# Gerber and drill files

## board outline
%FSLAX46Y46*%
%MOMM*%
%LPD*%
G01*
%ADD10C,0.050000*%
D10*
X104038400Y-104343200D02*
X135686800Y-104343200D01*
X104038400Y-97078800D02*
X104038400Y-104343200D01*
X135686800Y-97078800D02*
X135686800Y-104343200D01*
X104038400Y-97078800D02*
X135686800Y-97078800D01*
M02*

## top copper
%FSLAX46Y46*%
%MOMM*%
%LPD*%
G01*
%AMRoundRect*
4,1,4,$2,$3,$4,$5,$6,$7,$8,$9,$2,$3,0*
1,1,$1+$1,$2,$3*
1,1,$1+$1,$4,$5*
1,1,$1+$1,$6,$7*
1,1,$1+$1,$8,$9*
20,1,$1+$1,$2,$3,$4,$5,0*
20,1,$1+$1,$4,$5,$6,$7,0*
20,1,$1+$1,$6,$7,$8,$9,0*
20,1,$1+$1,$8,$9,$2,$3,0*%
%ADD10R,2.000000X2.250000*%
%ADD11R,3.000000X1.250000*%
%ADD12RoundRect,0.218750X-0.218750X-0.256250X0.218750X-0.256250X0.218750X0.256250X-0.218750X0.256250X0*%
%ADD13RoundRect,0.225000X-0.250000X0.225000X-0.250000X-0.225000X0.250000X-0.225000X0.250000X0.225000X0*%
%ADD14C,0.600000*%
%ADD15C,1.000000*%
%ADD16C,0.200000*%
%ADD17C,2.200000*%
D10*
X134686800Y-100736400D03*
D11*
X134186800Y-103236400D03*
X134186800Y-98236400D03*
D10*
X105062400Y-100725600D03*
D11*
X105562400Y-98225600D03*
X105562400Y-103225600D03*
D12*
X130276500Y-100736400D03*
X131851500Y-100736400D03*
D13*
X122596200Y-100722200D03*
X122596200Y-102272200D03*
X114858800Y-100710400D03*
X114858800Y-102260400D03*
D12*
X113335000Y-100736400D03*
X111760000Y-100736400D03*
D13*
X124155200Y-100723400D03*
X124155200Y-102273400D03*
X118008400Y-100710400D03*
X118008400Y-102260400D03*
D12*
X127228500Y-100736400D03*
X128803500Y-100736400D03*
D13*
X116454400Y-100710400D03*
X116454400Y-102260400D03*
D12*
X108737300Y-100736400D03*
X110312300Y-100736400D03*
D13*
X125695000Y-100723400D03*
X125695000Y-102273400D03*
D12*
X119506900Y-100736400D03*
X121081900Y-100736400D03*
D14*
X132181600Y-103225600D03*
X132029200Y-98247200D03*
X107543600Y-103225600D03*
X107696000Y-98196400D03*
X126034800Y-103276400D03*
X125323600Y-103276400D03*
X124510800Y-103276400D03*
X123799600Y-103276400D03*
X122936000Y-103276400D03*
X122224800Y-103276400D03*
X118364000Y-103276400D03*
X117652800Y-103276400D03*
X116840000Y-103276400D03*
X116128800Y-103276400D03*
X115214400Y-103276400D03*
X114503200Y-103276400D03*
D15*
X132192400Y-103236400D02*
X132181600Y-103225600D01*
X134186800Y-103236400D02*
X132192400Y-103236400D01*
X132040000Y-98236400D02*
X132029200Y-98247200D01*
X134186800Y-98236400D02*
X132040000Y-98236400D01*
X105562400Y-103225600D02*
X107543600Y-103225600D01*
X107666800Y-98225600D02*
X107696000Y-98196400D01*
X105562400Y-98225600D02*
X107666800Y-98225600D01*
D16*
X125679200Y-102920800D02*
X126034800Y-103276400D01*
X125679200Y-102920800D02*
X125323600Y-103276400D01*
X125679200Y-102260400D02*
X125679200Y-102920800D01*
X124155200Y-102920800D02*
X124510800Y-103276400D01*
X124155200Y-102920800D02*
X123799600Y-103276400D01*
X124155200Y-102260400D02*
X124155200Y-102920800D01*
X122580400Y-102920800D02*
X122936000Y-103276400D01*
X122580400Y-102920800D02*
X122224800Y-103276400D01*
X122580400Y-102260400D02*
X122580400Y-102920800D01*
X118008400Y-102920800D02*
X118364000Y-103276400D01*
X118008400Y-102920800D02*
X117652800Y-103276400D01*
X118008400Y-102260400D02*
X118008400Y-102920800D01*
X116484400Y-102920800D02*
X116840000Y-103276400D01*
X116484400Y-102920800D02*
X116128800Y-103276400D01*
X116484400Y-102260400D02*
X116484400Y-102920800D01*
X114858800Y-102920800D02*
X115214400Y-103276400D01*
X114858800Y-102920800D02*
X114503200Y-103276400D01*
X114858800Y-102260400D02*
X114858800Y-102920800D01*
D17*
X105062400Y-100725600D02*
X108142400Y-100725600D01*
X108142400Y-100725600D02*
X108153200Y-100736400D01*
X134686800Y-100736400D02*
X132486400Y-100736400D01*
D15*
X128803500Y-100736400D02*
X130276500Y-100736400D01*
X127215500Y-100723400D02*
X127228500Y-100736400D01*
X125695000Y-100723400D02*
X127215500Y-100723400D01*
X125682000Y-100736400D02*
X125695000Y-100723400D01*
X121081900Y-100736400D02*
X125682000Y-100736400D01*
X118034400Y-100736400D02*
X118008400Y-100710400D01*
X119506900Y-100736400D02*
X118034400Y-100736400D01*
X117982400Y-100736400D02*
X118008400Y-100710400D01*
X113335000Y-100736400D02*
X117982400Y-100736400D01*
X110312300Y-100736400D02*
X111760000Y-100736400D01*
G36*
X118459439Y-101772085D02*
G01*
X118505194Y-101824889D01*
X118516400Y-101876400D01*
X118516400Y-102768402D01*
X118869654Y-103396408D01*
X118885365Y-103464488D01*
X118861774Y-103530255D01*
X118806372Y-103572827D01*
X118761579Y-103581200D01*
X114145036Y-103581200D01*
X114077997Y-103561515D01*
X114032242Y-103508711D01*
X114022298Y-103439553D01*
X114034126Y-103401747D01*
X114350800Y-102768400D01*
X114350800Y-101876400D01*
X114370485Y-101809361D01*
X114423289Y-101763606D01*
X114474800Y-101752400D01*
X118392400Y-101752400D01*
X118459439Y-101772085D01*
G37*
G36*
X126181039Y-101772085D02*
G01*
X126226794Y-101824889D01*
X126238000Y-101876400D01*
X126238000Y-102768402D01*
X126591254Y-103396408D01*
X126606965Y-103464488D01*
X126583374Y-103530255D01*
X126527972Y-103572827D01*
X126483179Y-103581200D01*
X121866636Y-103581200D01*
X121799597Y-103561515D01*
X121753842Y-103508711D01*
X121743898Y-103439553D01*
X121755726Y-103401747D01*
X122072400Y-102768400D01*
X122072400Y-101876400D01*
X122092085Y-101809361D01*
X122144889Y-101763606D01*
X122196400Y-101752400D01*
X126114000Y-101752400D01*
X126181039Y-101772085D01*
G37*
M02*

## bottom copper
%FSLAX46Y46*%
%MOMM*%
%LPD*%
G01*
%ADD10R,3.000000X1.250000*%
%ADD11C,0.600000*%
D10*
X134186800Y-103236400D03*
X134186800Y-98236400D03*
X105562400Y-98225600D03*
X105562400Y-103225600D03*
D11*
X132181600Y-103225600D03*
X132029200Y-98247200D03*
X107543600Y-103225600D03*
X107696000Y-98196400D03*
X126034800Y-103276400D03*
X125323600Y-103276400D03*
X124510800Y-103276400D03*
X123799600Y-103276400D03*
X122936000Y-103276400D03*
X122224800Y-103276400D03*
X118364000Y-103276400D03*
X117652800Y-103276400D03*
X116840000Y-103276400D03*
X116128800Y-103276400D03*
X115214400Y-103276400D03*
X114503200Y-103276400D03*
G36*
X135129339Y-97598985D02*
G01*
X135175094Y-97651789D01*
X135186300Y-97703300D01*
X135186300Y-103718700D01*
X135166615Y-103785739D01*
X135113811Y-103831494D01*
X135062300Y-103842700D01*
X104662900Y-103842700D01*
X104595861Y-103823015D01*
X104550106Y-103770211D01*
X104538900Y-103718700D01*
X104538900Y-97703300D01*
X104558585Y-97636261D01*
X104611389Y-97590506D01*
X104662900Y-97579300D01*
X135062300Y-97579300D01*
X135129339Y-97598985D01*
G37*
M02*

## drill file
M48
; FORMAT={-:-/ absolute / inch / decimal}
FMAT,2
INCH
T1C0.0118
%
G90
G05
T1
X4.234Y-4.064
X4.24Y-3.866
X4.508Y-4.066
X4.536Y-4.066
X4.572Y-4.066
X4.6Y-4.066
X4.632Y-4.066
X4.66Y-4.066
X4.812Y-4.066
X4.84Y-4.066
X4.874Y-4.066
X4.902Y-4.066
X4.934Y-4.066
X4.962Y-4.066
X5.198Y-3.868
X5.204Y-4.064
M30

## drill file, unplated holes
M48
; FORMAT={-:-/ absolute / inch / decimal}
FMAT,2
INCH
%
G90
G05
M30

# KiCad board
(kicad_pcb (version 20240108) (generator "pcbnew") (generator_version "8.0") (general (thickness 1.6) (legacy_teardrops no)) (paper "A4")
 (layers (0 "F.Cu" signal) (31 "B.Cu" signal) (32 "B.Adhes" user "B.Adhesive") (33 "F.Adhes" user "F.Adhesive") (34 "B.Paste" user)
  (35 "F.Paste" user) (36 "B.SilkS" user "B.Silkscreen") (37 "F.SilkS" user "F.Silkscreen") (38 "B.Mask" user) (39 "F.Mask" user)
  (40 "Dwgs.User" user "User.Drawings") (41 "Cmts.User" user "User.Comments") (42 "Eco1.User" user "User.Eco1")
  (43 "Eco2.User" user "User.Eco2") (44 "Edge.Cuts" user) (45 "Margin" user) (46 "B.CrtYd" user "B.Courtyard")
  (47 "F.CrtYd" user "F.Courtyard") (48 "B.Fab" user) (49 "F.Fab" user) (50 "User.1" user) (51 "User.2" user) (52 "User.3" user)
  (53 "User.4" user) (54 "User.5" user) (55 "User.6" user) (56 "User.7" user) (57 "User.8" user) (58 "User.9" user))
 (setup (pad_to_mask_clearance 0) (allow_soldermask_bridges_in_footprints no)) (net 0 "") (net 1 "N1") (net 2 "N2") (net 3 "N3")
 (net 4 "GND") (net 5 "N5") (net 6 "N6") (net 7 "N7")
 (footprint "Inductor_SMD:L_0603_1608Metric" (layer "F.Cu") (at 131.064 100.7364)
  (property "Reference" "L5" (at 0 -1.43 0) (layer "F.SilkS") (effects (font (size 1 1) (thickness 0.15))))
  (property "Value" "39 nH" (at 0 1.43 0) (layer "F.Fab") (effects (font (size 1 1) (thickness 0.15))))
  (pad "1" smd roundrect (at -0.7875 0) (size 0.875 0.95) (layers "F.Cu" "F.Paste" "F.Mask") (roundrect_rratio 0.25) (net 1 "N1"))
  (pad "2" smd roundrect (at 0.7875 0) (size 0.875 0.95) (layers "F.Cu" "F.Paste" "F.Mask") (roundrect_rratio 0.25) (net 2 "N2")))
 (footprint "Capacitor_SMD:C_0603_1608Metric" (layer "F.Cu") (at 122.5962 101.4972 -90)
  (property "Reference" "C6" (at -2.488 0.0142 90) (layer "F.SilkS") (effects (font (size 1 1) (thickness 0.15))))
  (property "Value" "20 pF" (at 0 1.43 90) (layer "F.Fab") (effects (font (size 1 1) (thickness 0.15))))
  (pad "1" smd roundrect (at -0.775 0 270) (size 0.9 0.95) (layers "F.Cu" "F.Paste" "F.Mask") (roundrect_rratio 0.25) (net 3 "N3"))
  (pad "2" smd roundrect (at 0.775 0 270) (size 0.9 0.95) (layers "F.Cu" "F.Paste" "F.Mask") (roundrect_rratio 0.25) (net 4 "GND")))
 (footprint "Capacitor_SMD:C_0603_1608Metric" (layer "F.Cu") (at 114.8588 101.4854 -90)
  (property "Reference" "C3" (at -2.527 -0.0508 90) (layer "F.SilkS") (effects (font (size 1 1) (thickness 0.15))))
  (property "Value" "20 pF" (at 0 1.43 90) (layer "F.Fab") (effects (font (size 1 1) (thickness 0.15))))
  (pad "1" smd roundrect (at -0.775 0 270) (size 0.9 0.95) (layers "F.Cu" "F.Paste" "F.Mask") (roundrect_rratio 0.25) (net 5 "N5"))
  (pad "2" smd roundrect (at 0.775 0 270) (size 0.9 0.95) (layers "F.Cu" "F.Paste" "F.Mask") (roundrect_rratio 0.25) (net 4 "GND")))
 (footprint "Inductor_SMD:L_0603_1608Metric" (layer "F.Cu") (at 112.5475 100.7364)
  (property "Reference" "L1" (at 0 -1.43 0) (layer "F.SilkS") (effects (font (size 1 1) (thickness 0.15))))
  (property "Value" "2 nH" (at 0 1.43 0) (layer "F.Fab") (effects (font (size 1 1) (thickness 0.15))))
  (pad "1" smd roundrect (at -0.7875 0) (size 0.875 0.95) (layers "F.Cu" "F.Paste" "F.Mask") (roundrect_rratio 0.25) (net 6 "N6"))
  (pad "2" smd roundrect (at 0.7875 0) (size 0.875 0.95) (layers "F.Cu" "F.Paste" "F.Mask") (roundrect_rratio 0.25) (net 5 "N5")))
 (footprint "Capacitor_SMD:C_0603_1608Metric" (layer "F.Cu") (at 124.1552 101.4984 -90)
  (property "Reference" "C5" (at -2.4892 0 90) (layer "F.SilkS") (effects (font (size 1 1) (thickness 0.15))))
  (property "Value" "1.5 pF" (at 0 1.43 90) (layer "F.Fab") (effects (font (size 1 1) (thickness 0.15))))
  (pad "1" smd roundrect (at -0.775 0 270) (size 0.9 0.95) (layers "F.Cu" "F.Paste" "F.Mask") (roundrect_rratio 0.25) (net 3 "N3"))
  (pad "2" smd roundrect (at 0.775 0 270) (size 0.9 0.95) (layers "F.Cu" "F.Paste" "F.Mask") (roundrect_rratio 0.25) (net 4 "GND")))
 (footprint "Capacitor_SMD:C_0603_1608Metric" (layer "F.Cu") (at 118.0084 101.4854 -90)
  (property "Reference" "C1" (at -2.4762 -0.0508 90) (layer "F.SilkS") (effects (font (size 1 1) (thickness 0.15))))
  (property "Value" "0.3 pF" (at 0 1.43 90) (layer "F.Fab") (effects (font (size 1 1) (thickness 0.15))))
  (pad "1" smd roundrect (at -0.775 0 270) (size 0.9 0.95) (layers "F.Cu" "F.Paste" "F.Mask") (roundrect_rratio 0.25) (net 5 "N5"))
  (pad "2" smd roundrect (at 0.775 0 270) (size 0.9 0.95) (layers "F.Cu" "F.Paste" "F.Mask") (roundrect_rratio 0.25) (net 4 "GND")))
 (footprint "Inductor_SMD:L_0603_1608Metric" (layer "F.Cu") (at 128.016 100.7364)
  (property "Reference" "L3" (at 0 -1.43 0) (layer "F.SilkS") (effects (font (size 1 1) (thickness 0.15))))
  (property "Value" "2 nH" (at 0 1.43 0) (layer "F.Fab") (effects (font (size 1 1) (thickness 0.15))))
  (pad "1" smd roundrect (at -0.7875 0) (size 0.875 0.95) (layers "F.Cu" "F.Paste" "F.Mask") (roundrect_rratio 0.25) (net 3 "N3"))
  (pad "2" smd roundrect (at 0.7875 0) (size 0.875 0.95) (layers "F.Cu" "F.Paste" "F.Mask") (roundrect_rratio 0.25) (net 1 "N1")))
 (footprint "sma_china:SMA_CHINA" (layer "F.Cu") (at 135.6868 100.7364 90)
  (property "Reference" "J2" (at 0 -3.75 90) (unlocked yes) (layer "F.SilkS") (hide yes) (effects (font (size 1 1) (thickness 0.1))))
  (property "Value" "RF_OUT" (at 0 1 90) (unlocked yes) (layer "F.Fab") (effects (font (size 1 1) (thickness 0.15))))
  (pad "1" smd rect (at 0 -1 90) (size 2.25 2) (layers "F.Cu" "F.Paste" "F.Mask") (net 2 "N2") (thermal_bridge_angle 45))
  (pad "2" smd rect (at -2.5 -1.5 90) (size 1.25 3) (layers "F.Cu" "F.Paste" "F.Mask") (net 4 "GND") (thermal_bridge_angle 45))
  (pad "2" smd rect (at -2.5 -1.5 90) (size 1.25 3) (layers "B.Cu" "B.Paste" "B.Mask") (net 4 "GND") (thermal_bridge_angle 45))
  (pad "2" smd rect (at 2.5 -1.5 90) (size 1.25 3) (layers "F.Cu" "F.Paste" "F.Mask") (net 4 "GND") (thermal_bridge_angle 45))
  (pad "2" smd rect (at 2.5 -1.5 90) (size 1.25 3) (layers "B.Cu" "B.Paste" "B.Mask") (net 4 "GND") (thermal_bridge_angle 45)))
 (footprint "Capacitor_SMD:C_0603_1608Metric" (layer "F.Cu") (at 116.4544 101.4854 -90)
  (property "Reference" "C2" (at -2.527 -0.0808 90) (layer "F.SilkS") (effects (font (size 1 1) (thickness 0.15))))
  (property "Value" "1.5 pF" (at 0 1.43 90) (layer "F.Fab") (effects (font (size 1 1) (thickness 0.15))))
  (pad "1" smd roundrect (at -0.775 0 270) (size 0.9 0.95) (layers "F.Cu" "F.Paste" "F.Mask") (roundrect_rratio 0.25) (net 5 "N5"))
  (pad "2" smd roundrect (at 0.775 0 270) (size 0.9 0.95) (layers "F.Cu" "F.Paste" "F.Mask") (roundrect_rratio 0.25) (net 4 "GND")))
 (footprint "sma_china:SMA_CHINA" (layer "F.Cu") (at 104.0624 100.7256 -90)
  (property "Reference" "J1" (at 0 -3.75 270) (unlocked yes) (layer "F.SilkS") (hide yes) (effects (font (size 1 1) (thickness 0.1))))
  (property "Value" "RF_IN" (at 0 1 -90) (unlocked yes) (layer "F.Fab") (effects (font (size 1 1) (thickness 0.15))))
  (pad "1" smd rect (at 0 -1 270) (size 2.25 2) (layers "F.Cu" "F.Paste" "F.Mask") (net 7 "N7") (thermal_bridge_angle 45))
  (pad "2" smd rect (at -2.5 -1.5 270) (size 1.25 3) (layers "F.Cu" "F.Paste" "F.Mask") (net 4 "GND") (thermal_bridge_angle 45))
  (pad "2" smd rect (at -2.5 -1.5 270) (size 1.25 3) (layers "B.Cu" "B.Paste" "B.Mask") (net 4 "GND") (thermal_bridge_angle 45))
  (pad "2" smd rect (at 2.5 -1.5 270) (size 1.25 3) (layers "F.Cu" "F.Paste" "F.Mask") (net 4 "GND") (thermal_bridge_angle 45))
  (pad "2" smd rect (at 2.5 -1.5 270) (size 1.25 3) (layers "B.Cu" "B.Paste" "B.Mask") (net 4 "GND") (thermal_bridge_angle 45)))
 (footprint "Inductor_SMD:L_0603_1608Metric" (layer "F.Cu") (at 109.5248 100.7364)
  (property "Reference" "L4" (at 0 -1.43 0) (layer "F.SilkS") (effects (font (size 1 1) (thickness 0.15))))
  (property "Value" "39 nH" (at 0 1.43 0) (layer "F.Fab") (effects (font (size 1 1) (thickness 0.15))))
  (pad "1" smd roundrect (at -0.7875 0) (size 0.875 0.95) (layers "F.Cu" "F.Paste" "F.Mask") (roundrect_rratio 0.25) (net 7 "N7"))
  (pad "2" smd roundrect (at 0.7875 0) (size 0.875 0.95) (layers "F.Cu" "F.Paste" "F.Mask") (roundrect_rratio 0.25) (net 6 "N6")))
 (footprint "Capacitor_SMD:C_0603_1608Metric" (layer "F.Cu") (at 125.695 101.4984 -90)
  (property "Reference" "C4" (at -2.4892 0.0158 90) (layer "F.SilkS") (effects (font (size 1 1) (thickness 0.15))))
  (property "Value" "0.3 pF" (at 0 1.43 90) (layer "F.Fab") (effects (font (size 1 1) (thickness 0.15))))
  (pad "1" smd roundrect (at -0.775 0 270) (size 0.9 0.95) (layers "F.Cu" "F.Paste" "F.Mask") (roundrect_rratio 0.25) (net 3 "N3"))
  (pad "2" smd roundrect (at 0.775 0 270) (size 0.9 0.95) (layers "F.Cu" "F.Paste" "F.Mask") (roundrect_rratio 0.25) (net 4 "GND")))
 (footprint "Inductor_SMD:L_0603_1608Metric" (layer "F.Cu") (at 120.2944 100.7364)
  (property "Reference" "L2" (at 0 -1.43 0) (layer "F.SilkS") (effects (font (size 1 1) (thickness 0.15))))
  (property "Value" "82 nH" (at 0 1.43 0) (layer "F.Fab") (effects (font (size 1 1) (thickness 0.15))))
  (pad "1" smd roundrect (at -0.7875 0) (size 0.875 0.95) (layers "F.Cu" "F.Paste" "F.Mask") (roundrect_rratio 0.25) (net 5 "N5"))
  (pad "2" smd roundrect (at 0.7875 0) (size 0.875 0.95) (layers "F.Cu" "F.Paste" "F.Mask") (roundrect_rratio 0.25) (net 3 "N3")))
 (gr_line (start 135.6868 97.0788) (end 135.6868 104.3432) (stroke (width 0.05) (type default)) (layer "Edge.Cuts"))
 (gr_line (start 104.0384 97.0788) (end 104.0384 104.3432) (stroke (width 0.05) (type default)) (layer "Edge.Cuts"))
 (gr_line (start 104.0384 104.3432) (end 135.6868 104.3432) (stroke (width 0.05) (type default)) (layer "Edge.Cuts"))
 (gr_line (start 104.0384 97.0788) (end 135.6868 97.0788) (stroke (width 0.05) (type default)) (layer "Edge.Cuts"))
 (segment (start 105.5624 103.2256) (end 107.5436 103.2256) (width 1) (layer "F.Cu") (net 4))
 (segment (start 105.5624 98.2256) (end 107.6668 98.2256) (width 1) (layer "F.Cu") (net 4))
 (segment (start 116.4844 102.9208) (end 116.84 103.2764) (width 0.2) (layer "F.Cu") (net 4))
 (segment (start 124.1552 102.2604) (end 124.1552 102.9208) (width 0.2) (layer "F.Cu") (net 4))
 (segment (start 116.4844 102.9208) (end 116.1288 103.2764) (width 0.2) (layer "F.Cu") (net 4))
 (segment (start 132.1924 103.2364) (end 132.1816 103.2256) (width 1) (layer "F.Cu") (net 4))
 (segment (start 124.1552 102.9208) (end 123.7996 103.2764) (width 0.2) (layer "F.Cu") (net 4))
 (segment (start 107.6668 98.2256) (end 107.696 98.1964) (width 1) (layer "F.Cu") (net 4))
 (segment (start 114.8588 102.9208) (end 114.5032 103.2764) (width 0.2) (layer "F.Cu") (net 4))
 (segment (start 118.0084 102.2604) (end 118.0084 102.9208) (width 0.2) (layer "F.Cu") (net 4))
 (segment (start 124.1552 102.9208) (end 124.5108 103.2764) (width 0.2) (layer "F.Cu") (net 4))
 (segment (start 118.0084 102.9208) (end 117.6528 103.2764) (width 0.2) (layer "F.Cu") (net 4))
 (segment (start 125.6792 102.2604) (end 125.6792 102.9208) (width 0.2) (layer "F.Cu") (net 4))
 (segment (start 122.5804 102.2604) (end 122.5804 102.9208) (width 0.2) (layer "F.Cu") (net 4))
 (segment (start 125.6792 102.9208) (end 125.3236 103.2764) (width 0.2) (layer "F.Cu") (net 4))
 (segment (start 114.8588 102.9208) (end 115.2144 103.2764) (width 0.2) (layer "F.Cu") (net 4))
 (segment (start 122.5804 102.9208) (end 122.2248 103.2764) (width 0.2) (layer "F.Cu") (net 4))
 (segment (start 114.8588 102.2604) (end 114.8588 102.9208) (width 0.2) (layer "F.Cu") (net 4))
 (segment (start 116.4844 102.2604) (end 116.4844 102.9208) (width 0.2) (layer "F.Cu") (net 4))
 (segment (start 125.6792 102.9208) (end 126.0348 103.2764) (width 0.2) (layer "F.Cu") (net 4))
 (segment (start 122.5804 102.9208) (end 122.936 103.2764) (width 0.2) (layer "F.Cu") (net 4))
 (segment (start 134.1868 98.2364) (end 132.04 98.2364) (width 1) (layer "F.Cu") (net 4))
 (segment (start 134.1868 103.2364) (end 132.1924 103.2364) (width 1) (layer "F.Cu") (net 4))
 (segment (start 118.0084 102.9208) (end 118.364 103.2764) (width 0.2) (layer "F.Cu") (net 4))
 (segment (start 132.04 98.2364) (end 132.0292 98.2472) (width 1) (layer "F.Cu") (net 4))
 (via (at 118.364 103.2764) (size 0.6) (drill 0.3) (layers "F.Cu" "B.Cu") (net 4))
 (via (at 116.84 103.2764) (size 0.6) (drill 0.3) (layers "F.Cu" "B.Cu") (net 4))
 (via (at 117.6528 103.2764) (size 0.6) (drill 0.3) (layers "F.Cu" "B.Cu") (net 4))
 (via (at 116.1288 103.2764) (size 0.6) (drill 0.3) (layers "F.Cu" "B.Cu") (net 4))
 (via (at 132.1816 103.2256) (size 0.6) (drill 0.3) (layers "F.Cu" "B.Cu") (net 4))
 (via (at 124.5108 103.2764) (size 0.6) (drill 0.3) (layers "F.Cu" "B.Cu") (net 4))
 (via (at 114.5032 103.2764) (size 0.6) (drill 0.3) (layers "F.Cu" "B.Cu") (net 4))
 (via (at 122.936 103.2764) (size 0.6) (drill 0.3) (layers "F.Cu" "B.Cu") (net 4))
 (via (at 125.3236 103.2764) (size 0.6) (drill 0.3) (layers "F.Cu" "B.Cu") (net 4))
 (via (at 122.2248 103.2764) (size 0.6) (drill 0.3) (layers "F.Cu" "B.Cu") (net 4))
 (via (at 107.696 98.1964) (size 0.6) (drill 0.3) (layers "F.Cu" "B.Cu") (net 4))
 (via (at 132.0292 98.2472) (size 0.6) (drill 0.3) (layers "F.Cu" "B.Cu") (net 4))
 (via (at 123.7996 103.2764) (size 0.6) (drill 0.3) (layers "F.Cu" "B.Cu") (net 4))
 (via (at 126.0348 103.2764) (size 0.6) (drill 0.3) (layers "F.Cu" "B.Cu") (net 4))
 (via (at 107.5436 103.2256) (size 0.6) (drill 0.3) (layers "F.Cu" "B.Cu") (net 4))
 (via (at 115.2144 103.2764) (size 0.6) (drill 0.3) (layers "F.Cu" "B.Cu") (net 4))
 (segment (start 113.335 100.7364) (end 117.9824 100.7364) (width 1) (layer "F.Cu") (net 5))
 (segment (start 119.5069 100.7364) (end 118.0344 100.7364) (width 1) (layer "F.Cu") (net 5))
 (segment (start 117.9824 100.7364) (end 118.0084 100.7104) (width 1) (layer "F.Cu") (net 5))
 (segment (start 118.0344 100.7364) (end 118.0084 100.7104) (width 1) (layer "F.Cu") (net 5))
 (segment (start 125.695 100.7234) (end 127.2155 100.7234) (width 1) (layer "F.Cu") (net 3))
 (segment (start 125.682 100.7364) (end 125.695 100.7234) (width 1) (layer "F.Cu") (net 3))
 (segment (start 121.0819 100.7364) (end 125.682 100.7364) (width 1) (layer "F.Cu") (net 3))
 (segment (start 127.2155 100.7234) (end 127.2285 100.7364) (width 1) (layer "F.Cu") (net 3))
 (segment (start 105.0624 100.7256) (end 108.1424 100.7256) (width 2.2) (layer "F.Cu") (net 7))
 (segment (start 108.1424 100.7256) (end 108.1532 100.7364) (width 2.2) (layer "F.Cu") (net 7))
 (segment (start 134.6868 100.7364) (end 132.4864 100.7364) (width 2.2) (layer "F.Cu") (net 2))
 (segment (start 110.3123 100.7364) (end 111.76 100.7364) (width 1) (layer "F.Cu") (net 6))
 (segment (start 128.8035 100.7364) (end 130.2765 100.7364) (width 1) (layer "F.Cu") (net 1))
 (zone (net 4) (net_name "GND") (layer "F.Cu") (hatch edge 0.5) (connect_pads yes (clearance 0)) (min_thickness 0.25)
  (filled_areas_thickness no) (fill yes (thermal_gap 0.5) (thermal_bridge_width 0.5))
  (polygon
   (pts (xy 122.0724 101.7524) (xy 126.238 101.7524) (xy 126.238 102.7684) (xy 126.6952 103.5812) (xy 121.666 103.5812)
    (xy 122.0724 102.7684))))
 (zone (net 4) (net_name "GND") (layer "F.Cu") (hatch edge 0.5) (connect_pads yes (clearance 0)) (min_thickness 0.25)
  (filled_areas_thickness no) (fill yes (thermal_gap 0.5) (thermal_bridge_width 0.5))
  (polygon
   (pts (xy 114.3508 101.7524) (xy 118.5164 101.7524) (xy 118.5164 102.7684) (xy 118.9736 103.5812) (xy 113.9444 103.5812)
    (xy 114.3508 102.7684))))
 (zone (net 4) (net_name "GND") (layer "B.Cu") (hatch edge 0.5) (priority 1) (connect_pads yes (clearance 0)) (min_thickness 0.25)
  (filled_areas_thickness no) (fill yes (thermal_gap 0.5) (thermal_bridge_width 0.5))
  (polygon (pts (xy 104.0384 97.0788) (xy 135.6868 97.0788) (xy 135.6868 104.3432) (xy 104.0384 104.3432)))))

